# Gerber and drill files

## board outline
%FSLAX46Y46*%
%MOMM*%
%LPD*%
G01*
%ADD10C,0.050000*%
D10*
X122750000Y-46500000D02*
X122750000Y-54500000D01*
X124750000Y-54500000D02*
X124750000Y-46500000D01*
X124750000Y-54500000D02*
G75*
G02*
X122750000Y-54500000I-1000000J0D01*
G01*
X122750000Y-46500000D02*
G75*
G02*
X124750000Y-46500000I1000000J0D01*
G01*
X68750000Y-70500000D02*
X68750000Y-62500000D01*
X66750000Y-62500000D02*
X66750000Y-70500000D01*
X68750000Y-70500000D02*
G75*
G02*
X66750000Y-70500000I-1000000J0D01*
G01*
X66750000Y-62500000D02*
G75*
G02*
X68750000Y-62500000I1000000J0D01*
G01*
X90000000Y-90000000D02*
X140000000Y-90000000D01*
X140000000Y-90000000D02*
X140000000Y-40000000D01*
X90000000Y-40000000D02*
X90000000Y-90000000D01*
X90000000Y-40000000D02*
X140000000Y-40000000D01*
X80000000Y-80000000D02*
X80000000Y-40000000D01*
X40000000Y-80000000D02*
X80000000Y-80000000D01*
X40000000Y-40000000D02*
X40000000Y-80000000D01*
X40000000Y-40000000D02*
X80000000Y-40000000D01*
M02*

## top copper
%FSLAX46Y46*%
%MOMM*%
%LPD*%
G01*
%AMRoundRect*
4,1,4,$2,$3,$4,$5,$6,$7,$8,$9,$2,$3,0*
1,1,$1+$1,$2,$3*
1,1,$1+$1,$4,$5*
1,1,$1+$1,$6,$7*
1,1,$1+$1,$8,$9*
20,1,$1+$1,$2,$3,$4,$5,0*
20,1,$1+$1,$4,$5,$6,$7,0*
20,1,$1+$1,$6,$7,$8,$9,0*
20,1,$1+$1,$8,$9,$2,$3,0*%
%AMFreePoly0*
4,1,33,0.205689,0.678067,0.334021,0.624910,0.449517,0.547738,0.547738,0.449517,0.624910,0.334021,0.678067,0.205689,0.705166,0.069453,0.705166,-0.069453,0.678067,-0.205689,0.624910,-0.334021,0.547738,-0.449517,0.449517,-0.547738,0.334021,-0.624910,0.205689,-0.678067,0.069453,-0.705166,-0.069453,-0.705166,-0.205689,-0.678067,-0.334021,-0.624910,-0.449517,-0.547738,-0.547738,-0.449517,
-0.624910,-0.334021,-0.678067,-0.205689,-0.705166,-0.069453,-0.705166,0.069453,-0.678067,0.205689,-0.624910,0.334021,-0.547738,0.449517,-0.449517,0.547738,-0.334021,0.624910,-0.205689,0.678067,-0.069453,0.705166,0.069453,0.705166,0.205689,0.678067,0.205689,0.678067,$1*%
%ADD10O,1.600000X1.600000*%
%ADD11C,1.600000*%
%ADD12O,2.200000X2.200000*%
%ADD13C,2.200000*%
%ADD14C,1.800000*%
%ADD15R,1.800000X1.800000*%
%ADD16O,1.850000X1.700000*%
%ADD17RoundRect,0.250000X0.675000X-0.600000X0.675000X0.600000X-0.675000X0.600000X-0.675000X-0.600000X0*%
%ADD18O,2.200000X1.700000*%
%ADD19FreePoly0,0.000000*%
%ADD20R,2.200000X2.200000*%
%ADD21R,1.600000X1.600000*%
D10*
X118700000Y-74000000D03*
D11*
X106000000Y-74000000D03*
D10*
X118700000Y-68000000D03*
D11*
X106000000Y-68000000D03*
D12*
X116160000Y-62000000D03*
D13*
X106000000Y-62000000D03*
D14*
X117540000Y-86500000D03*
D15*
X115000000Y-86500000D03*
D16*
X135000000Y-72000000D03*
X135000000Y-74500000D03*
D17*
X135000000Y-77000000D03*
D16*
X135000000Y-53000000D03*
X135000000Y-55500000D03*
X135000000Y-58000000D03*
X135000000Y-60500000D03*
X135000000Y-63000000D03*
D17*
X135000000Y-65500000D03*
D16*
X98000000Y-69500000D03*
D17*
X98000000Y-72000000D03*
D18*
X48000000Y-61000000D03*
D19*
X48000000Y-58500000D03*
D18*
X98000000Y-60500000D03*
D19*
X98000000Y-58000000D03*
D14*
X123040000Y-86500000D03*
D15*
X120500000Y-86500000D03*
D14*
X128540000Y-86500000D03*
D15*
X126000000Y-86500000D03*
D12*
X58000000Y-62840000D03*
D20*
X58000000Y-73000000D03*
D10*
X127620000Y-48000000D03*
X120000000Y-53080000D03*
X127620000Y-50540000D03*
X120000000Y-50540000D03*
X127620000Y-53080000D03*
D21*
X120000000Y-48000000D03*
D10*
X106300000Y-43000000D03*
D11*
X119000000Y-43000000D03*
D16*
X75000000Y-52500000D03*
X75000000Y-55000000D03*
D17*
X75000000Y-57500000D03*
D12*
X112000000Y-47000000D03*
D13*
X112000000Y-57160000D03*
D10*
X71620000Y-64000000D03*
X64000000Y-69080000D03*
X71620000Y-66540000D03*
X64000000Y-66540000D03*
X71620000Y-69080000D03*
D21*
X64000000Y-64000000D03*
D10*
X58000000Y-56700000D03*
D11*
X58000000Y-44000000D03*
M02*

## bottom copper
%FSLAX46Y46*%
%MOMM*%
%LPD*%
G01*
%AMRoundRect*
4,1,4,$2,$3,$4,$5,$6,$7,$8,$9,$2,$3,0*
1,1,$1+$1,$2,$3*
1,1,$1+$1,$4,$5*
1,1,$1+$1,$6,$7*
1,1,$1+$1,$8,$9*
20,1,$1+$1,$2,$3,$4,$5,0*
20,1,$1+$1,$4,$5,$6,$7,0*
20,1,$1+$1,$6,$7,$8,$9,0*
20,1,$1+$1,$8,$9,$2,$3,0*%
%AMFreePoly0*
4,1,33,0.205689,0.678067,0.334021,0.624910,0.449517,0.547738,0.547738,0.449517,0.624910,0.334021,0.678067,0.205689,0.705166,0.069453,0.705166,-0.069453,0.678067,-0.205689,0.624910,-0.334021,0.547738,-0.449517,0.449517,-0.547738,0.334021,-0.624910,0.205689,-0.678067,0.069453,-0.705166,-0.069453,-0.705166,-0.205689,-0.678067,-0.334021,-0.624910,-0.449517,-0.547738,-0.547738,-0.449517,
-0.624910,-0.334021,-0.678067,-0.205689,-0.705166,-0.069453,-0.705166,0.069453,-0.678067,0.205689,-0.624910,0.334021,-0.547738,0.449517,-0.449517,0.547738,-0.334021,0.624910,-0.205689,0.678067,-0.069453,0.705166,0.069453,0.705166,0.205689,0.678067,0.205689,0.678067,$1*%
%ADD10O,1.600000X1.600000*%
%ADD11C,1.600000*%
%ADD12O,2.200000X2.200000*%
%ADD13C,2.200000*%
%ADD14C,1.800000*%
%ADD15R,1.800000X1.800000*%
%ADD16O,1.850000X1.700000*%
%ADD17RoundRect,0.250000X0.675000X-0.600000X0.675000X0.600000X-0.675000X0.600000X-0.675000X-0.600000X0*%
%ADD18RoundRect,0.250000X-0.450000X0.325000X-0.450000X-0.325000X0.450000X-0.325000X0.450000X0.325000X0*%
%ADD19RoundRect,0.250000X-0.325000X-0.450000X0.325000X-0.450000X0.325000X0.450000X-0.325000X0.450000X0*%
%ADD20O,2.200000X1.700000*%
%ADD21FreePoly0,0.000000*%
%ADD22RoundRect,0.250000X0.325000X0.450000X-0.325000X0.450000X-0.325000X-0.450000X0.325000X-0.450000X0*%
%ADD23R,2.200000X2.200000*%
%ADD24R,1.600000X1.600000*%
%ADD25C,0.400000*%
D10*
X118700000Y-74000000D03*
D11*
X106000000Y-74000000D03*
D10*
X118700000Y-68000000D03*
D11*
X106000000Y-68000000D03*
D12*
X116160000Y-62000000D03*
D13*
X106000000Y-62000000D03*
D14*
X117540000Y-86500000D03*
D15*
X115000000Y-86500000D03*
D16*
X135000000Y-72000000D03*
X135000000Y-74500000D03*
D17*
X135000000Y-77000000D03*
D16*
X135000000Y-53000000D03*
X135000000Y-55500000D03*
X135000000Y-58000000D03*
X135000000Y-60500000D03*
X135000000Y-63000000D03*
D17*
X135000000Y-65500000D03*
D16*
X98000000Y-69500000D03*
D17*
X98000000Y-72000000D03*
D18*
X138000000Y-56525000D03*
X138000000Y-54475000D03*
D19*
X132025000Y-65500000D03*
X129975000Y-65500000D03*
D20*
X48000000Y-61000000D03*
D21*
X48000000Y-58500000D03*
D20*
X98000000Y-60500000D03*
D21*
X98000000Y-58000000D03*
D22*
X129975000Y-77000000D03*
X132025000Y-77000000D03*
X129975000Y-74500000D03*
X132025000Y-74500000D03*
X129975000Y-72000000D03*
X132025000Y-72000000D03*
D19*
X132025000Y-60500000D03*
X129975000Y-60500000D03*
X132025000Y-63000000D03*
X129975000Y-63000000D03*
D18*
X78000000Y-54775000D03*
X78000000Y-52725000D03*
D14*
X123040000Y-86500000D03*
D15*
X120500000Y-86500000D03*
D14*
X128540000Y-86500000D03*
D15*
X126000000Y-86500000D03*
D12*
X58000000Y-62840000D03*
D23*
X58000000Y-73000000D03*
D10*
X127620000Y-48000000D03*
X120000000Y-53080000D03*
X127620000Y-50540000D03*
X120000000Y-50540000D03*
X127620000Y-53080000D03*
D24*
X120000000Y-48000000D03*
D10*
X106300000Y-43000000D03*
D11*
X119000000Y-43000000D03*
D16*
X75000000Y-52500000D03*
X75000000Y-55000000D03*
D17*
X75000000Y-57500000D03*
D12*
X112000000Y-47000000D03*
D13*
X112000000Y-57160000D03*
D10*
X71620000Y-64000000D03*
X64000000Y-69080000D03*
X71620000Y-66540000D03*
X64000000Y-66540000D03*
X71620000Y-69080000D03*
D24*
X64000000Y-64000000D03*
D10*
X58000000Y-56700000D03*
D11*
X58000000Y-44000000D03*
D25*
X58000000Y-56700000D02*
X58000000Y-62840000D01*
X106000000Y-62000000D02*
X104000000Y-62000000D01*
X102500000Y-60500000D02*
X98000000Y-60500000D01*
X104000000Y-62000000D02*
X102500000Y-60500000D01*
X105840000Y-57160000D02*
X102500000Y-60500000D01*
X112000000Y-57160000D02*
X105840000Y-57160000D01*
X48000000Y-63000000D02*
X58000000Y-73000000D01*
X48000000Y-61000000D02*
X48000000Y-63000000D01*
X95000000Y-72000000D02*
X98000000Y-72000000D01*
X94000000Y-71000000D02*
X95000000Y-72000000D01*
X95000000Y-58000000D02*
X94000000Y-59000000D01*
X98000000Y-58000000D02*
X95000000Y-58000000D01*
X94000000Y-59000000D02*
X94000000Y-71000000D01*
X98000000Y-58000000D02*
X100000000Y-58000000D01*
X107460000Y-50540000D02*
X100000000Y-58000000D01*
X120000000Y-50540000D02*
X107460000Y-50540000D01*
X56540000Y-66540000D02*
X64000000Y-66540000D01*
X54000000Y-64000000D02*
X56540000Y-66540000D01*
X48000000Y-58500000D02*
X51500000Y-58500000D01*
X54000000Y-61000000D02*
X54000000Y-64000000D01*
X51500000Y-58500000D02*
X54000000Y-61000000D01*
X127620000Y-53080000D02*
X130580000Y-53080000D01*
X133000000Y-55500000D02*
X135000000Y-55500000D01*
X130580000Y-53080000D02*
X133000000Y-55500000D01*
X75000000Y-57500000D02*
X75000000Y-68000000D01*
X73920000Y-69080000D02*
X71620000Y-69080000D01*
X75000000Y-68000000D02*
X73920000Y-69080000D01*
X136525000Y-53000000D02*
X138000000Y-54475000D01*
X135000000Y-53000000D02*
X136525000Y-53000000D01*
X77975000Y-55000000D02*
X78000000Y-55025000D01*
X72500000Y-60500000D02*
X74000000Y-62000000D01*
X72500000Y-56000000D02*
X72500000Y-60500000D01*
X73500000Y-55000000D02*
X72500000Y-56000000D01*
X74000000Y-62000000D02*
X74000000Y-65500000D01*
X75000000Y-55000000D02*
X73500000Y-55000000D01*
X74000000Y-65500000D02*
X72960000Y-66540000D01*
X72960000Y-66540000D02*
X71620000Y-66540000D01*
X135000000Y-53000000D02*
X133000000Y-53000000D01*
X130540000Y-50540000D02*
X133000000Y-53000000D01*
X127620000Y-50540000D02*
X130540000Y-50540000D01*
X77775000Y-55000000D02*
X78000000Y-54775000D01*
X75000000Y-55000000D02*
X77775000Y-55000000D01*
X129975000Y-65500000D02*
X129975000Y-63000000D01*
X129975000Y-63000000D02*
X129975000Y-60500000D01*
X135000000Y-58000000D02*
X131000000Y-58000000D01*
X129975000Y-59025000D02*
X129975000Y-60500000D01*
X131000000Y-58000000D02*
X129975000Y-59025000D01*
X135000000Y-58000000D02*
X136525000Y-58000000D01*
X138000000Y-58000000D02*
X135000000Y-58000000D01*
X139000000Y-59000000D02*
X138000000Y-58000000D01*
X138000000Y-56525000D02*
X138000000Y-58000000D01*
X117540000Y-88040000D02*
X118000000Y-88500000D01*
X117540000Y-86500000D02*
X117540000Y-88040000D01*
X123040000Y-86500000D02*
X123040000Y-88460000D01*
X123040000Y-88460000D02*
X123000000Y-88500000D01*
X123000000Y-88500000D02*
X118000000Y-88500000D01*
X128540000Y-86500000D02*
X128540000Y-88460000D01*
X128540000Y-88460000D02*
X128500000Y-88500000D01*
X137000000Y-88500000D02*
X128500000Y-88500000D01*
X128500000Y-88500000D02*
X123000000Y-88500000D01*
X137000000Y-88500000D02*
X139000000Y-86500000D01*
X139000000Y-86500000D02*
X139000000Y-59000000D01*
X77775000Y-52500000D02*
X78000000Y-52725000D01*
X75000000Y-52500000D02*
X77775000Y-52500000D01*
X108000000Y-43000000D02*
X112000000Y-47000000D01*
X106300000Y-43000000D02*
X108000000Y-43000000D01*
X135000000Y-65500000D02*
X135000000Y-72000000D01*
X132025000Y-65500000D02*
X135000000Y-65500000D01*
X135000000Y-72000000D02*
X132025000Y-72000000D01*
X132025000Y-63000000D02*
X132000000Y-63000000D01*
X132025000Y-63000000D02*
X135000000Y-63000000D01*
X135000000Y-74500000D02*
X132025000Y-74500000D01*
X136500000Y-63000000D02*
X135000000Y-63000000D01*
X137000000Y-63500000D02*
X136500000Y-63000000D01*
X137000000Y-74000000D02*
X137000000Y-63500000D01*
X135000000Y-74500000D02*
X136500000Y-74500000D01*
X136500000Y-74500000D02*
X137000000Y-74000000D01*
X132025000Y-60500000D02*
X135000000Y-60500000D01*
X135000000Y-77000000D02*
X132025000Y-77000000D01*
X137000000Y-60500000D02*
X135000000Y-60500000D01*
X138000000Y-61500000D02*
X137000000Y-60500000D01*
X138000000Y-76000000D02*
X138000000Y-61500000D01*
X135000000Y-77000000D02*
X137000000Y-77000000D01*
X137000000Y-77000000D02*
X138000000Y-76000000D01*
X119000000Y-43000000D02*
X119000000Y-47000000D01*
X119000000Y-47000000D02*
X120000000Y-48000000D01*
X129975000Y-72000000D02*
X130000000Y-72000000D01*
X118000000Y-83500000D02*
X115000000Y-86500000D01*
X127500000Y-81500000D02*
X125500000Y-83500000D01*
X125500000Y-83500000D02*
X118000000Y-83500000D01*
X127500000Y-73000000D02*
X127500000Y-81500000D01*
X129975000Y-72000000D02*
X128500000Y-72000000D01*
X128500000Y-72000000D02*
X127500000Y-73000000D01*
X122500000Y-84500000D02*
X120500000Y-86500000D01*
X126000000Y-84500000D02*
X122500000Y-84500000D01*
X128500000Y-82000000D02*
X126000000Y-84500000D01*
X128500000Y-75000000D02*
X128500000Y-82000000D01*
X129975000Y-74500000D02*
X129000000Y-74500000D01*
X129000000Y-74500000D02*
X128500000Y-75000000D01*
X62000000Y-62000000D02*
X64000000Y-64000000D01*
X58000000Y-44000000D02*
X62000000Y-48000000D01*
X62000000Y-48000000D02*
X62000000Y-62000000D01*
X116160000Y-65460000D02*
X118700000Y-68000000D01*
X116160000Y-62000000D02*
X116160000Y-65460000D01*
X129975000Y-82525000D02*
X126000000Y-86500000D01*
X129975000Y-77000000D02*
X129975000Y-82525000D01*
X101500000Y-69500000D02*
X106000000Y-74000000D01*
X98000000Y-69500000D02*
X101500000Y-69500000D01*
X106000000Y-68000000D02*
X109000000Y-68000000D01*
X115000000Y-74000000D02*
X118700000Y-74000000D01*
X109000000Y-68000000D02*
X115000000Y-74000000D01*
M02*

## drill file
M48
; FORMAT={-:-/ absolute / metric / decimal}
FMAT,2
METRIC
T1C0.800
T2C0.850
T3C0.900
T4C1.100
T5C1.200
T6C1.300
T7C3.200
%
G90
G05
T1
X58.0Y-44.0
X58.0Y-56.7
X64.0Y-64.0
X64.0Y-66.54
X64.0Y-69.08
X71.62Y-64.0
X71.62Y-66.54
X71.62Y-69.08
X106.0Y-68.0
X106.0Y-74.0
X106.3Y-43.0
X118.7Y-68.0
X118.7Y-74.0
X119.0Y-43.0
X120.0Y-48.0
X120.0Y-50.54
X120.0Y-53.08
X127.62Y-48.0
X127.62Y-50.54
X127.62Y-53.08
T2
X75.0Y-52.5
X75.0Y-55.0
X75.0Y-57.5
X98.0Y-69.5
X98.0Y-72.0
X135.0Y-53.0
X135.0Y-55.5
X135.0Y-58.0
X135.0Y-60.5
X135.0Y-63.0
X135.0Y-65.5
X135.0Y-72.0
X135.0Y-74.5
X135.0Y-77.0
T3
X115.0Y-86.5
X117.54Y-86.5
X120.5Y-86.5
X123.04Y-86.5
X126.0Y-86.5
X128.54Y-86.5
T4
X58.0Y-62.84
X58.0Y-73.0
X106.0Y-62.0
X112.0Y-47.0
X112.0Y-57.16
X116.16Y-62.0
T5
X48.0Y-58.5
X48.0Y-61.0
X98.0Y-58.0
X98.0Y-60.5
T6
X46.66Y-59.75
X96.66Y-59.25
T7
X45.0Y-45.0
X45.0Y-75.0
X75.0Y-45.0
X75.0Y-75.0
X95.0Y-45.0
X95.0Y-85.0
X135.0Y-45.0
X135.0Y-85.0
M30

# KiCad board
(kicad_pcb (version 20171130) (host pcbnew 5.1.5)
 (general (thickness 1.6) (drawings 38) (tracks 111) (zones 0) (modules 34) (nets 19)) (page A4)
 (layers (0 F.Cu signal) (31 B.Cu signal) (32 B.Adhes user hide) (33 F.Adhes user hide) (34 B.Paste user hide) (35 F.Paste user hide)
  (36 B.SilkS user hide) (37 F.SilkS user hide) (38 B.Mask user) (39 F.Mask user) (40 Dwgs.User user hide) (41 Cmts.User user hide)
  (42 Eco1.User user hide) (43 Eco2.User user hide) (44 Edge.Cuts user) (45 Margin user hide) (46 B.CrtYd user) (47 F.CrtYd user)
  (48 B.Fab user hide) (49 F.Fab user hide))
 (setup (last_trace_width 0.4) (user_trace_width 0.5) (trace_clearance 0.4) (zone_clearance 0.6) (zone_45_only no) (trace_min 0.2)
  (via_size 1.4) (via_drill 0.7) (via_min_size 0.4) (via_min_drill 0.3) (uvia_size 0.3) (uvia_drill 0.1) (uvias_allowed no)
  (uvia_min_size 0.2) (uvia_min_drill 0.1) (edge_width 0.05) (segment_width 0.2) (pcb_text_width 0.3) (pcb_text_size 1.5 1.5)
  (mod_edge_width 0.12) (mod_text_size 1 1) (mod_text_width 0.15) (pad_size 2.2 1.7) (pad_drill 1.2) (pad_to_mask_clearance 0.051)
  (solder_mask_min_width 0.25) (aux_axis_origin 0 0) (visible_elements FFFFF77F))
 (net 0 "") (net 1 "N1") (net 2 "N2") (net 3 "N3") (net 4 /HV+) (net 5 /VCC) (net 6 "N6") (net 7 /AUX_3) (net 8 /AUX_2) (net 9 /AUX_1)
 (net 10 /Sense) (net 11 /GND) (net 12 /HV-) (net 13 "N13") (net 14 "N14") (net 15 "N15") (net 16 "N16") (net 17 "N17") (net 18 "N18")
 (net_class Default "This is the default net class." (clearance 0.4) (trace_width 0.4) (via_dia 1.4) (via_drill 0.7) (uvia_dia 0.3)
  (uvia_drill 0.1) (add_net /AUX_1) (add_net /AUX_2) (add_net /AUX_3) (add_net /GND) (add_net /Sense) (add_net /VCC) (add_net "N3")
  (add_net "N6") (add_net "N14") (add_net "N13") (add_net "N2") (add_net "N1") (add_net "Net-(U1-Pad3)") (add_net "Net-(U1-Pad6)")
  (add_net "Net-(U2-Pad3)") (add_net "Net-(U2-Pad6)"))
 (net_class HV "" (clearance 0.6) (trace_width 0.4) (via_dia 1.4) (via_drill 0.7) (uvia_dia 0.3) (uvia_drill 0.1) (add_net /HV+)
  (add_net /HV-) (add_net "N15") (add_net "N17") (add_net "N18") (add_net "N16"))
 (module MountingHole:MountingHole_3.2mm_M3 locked (layer F.Cu) (at 45 45) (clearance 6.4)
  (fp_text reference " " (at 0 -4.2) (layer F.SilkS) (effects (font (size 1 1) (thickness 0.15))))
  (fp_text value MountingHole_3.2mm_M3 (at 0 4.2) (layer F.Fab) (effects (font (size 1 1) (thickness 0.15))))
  (pad 1 np_thru_hole circle (at 0 0) (size 3.2 3.2) (drill 3.2) (layers *.Cu *.Mask)))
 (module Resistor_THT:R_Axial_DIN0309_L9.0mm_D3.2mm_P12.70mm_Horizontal (layer F.Cu) (at 106 74)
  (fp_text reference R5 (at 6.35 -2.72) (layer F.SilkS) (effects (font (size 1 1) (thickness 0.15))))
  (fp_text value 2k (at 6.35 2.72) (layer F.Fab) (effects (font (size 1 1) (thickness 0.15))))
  (pad 2 thru_hole oval (at 12.7 0) (size 1.6 1.6) (drill 0.8) (layers *.Cu *.Mask) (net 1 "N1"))
  (pad 1 thru_hole circle (at 0 0) (size 1.6 1.6) (drill 0.8) (layers *.Cu *.Mask) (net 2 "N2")))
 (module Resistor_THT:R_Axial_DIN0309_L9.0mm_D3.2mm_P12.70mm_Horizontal (layer F.Cu) (at 106 68)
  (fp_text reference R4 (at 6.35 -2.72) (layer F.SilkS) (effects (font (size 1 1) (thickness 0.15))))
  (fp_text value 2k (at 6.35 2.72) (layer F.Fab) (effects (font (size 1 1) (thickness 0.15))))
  (pad 2 thru_hole oval (at 12.7 0) (size 1.6 1.6) (drill 0.8) (layers *.Cu *.Mask) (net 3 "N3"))
  (pad 1 thru_hole circle (at 0 0) (size 1.6 1.6) (drill 0.8) (layers *.Cu *.Mask) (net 1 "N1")))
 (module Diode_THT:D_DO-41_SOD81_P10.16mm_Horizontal (layer F.Cu) (at 106 62)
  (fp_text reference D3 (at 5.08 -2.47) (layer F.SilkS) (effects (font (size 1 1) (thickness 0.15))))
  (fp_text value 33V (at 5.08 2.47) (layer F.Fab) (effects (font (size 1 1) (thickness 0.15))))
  (pad 2 thru_hole oval (at 10.16 0) (size 2.2 2.2) (drill 1.1) (layers *.Cu *.Mask) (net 3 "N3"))
  (pad 1 thru_hole circle (at 0 0) (size 2.2 2.2) (drill 1.1) (layers *.Cu *.Mask) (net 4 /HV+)))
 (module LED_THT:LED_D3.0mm (layer F.Cu) (at 115 86.5)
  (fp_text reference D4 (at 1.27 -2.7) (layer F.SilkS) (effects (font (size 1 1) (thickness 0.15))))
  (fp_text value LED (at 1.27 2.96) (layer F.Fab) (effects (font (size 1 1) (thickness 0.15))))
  (pad 2 thru_hole circle (at 2.54 0) (size 1.8 1.8) (drill 0.9) (layers *.Cu *.Mask) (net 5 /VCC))
  (pad 1 thru_hole rect (at 0 0) (size 1.8 1.8) (drill 0.9) (layers *.Cu *.Mask) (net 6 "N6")))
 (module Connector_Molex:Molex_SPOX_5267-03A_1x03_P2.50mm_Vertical (layer F.Cu) (at 135 77 90)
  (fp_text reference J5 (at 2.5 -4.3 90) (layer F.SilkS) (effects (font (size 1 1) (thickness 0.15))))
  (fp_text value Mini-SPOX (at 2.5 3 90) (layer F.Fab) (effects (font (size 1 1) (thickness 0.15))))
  (pad 3 thru_hole oval (at 5 0 90) (size 1.7 1.85) (drill 0.85) (layers *.Cu *.Mask) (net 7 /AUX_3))
  (pad 2 thru_hole oval (at 2.5 0 90) (size 1.7 1.85) (drill 0.85) (layers *.Cu *.Mask) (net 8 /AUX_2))
  (pad 1 thru_hole roundrect (at 0 0 90) (size 1.7 1.85) (drill 0.85) (layers *.Cu *.Mask) (roundrect_rratio 0.147059) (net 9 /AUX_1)))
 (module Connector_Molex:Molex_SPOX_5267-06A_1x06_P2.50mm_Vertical (layer F.Cu) (at 135 65.5 90)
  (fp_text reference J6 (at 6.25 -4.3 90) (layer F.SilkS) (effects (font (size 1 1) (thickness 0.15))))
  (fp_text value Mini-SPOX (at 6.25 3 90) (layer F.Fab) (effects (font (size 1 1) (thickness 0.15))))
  (pad 6 thru_hole oval (at 12.5 0 90) (size 1.7 1.85) (drill 0.85) (layers *.Cu *.Mask) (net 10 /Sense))
  (pad 5 thru_hole oval (at 10 0 90) (size 1.7 1.85) (drill 0.85) (layers *.Cu *.Mask) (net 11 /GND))
  (pad 4 thru_hole oval (at 7.5 0 90) (size 1.7 1.85) (drill 0.85) (layers *.Cu *.Mask) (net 5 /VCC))
  (pad 3 thru_hole oval (at 5 0 90) (size 1.7 1.85) (drill 0.85) (layers *.Cu *.Mask) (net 9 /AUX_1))
  (pad 2 thru_hole oval (at 2.5 0 90) (size 1.7 1.85) (drill 0.85) (layers *.Cu *.Mask) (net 8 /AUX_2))
  (pad 1 thru_hole roundrect (at 0 0 90) (size 1.7 1.85) (drill 0.85) (layers *.Cu *.Mask) (roundrect_rratio 0.147059) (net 7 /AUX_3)))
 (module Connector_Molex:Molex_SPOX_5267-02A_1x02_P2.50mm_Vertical (layer F.Cu) (at 98 72 90)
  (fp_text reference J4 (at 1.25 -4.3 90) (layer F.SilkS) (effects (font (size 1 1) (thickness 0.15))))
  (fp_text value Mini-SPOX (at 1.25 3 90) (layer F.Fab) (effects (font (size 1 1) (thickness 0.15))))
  (pad 2 thru_hole oval (at 2.5 0 90) (size 1.7 1.85) (drill 0.85) (layers *.Cu *.Mask) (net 2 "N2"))
  (pad 1 thru_hole roundrect (at 0 0 90) (size 1.7 1.85) (drill 0.85) (layers *.Cu *.Mask) (roundrect_rratio 0.147059) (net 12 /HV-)))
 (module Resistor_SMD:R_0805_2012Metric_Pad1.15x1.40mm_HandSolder (layer B.Cu) (at 138 55.5 270)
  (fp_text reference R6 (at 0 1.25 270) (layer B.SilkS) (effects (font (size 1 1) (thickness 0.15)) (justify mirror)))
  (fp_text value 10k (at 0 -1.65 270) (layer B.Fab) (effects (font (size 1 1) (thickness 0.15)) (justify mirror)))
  (pad 2 smd roundrect (at 1.025 0 270) (size 1.15 1.4) (layers B.Cu B.Paste B.Mask) (roundrect_rratio 0.217391) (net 5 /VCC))
  (pad 1 smd roundrect (at -1.025 0 270) (size 1.15 1.4) (layers B.Cu B.Paste B.Mask) (roundrect_rratio 0.217391) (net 10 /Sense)))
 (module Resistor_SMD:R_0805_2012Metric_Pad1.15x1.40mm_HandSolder (layer B.Cu) (at 131 65.5)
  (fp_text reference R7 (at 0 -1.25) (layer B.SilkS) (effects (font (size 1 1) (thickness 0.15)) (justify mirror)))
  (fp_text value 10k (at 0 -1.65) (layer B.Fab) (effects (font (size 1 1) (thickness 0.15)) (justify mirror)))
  (pad 2 smd roundrect (at 1.025 0) (size 1.15 1.4) (layers B.Cu B.Paste B.Mask) (roundrect_rratio 0.217391) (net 7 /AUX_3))
  (pad 1 smd roundrect (at -1.025 0) (size 1.15 1.4) (layers B.Cu B.Paste B.Mask) (roundrect_rratio 0.217391) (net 5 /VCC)))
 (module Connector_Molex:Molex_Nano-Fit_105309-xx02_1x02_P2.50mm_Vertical (layer F.Cu) (at 48 58.5)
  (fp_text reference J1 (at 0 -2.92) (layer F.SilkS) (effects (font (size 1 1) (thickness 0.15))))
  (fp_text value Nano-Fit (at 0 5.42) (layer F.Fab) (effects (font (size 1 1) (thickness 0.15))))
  (pad "" np_thru_hole circle (at -1.34 1.25) (size 1.3 1.3) (drill 1.3) (layers *.Cu *.Mask))
  (pad 2 thru_hole oval (at 0 2.5) (size 2.2 1.7) (drill 1.2) (layers *.Cu *.Mask) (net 4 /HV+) (zone_connect 2))
  (pad 1 thru_hole custom (at 0 0) (size 1.417157 1.417157) (drill 1.2) (layers *.Cu *.Mask) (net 12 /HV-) (zone_connect 2)
   (options (clearance outline) (anchor circle)) (primitives)))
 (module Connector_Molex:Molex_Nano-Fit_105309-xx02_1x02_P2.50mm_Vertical (layer F.Cu) (at 98 58)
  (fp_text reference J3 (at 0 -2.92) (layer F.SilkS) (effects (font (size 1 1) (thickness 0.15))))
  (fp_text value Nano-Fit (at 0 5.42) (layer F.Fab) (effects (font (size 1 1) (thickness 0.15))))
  (pad "" np_thru_hole circle (at -1.34 1.25) (size 1.3 1.3) (drill 1.3) (layers *.Cu *.Mask))
  (pad 2 thru_hole oval (at 0 2.5) (size 2.2 1.7) (drill 1.2) (layers *.Cu *.Mask) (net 4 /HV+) (zone_connect 2))
  (pad 1 thru_hole custom (at 0 0) (size 1.417157 1.417157) (drill 1.2) (layers *.Cu *.Mask) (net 12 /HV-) (zone_connect 2)
   (options (clearance outline) (anchor circle)) (primitives)))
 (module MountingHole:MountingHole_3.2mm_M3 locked (layer F.Cu) (at 95 45) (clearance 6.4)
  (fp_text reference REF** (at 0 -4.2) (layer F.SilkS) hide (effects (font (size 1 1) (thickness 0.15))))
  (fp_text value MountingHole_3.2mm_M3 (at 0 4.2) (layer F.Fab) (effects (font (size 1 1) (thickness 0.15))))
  (pad 1 np_thru_hole circle (at 0 0) (size 3.2 3.2) (drill 3.2) (layers *.Cu *.Mask)))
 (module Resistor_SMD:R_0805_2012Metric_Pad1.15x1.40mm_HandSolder (layer B.Cu) (at 131 77 180)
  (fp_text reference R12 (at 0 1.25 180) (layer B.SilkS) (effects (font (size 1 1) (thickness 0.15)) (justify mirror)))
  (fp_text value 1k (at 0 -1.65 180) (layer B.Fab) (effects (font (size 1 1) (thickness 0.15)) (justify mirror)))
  (pad 2 smd roundrect (at 1.025 0 180) (size 1.15 1.4) (layers B.Cu B.Paste B.Mask) (roundrect_rratio 0.217391) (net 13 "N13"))
  (pad 1 smd roundrect (at -1.025 0 180) (size 1.15 1.4) (layers B.Cu B.Paste B.Mask) (roundrect_rratio 0.217391) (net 9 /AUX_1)))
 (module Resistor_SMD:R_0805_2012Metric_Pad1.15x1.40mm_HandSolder (layer B.Cu) (at 131 74.5 180)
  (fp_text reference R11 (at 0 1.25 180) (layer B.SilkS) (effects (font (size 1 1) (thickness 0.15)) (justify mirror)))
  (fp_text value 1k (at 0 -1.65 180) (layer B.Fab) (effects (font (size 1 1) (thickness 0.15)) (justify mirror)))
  (pad 2 smd roundrect (at 1.025 0 180) (size 1.15 1.4) (layers B.Cu B.Paste B.Mask) (roundrect_rratio 0.217391) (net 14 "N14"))
  (pad 1 smd roundrect (at -1.025 0 180) (size 1.15 1.4) (layers B.Cu B.Paste B.Mask) (roundrect_rratio 0.217391) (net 8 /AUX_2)))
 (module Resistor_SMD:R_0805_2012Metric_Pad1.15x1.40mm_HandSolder (layer B.Cu) (at 131 72 180)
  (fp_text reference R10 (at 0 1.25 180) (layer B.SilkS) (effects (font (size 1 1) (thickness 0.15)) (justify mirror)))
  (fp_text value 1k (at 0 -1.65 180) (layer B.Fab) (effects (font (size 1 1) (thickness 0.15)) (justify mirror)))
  (pad 2 smd roundrect (at 1.025 0 180) (size 1.15 1.4) (layers B.Cu B.Paste B.Mask) (roundrect_rratio 0.217391) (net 6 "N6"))
  (pad 1 smd roundrect (at -1.025 0 180) (size 1.15 1.4) (layers B.Cu B.Paste B.Mask) (roundrect_rratio 0.217391) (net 7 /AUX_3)))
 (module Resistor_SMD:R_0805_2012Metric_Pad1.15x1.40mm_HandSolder (layer B.Cu) (at 131 60.5)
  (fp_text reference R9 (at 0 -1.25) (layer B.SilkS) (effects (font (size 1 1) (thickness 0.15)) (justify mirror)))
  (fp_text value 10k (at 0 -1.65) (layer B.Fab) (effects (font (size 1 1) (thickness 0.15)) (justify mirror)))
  (pad 2 smd roundrect (at 1.025 0) (size 1.15 1.4) (layers B.Cu B.Paste B.Mask) (roundrect_rratio 0.217391) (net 9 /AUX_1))
  (pad 1 smd roundrect (at -1.025 0) (size 1.15 1.4) (layers B.Cu B.Paste B.Mask) (roundrect_rratio 0.217391) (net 5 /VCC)))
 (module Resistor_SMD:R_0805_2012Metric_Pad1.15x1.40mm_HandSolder (layer B.Cu) (at 131 63)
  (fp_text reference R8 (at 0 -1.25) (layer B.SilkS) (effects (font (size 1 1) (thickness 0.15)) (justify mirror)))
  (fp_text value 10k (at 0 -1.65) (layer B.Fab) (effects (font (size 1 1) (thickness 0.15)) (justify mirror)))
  (pad 2 smd roundrect (at 1.025 0) (size 1.15 1.4) (layers B.Cu B.Paste B.Mask) (roundrect_rratio 0.217391) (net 8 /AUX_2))
  (pad 1 smd roundrect (at -1.025 0) (size 1.15 1.4) (layers B.Cu B.Paste B.Mask) (roundrect_rratio 0.217391) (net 5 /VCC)))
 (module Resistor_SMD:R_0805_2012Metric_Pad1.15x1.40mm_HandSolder (layer B.Cu) (at 78 53.75 270)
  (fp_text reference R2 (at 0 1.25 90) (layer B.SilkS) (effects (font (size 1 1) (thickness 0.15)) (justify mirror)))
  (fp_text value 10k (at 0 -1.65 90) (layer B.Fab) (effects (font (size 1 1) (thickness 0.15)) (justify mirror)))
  (pad 2 smd roundrect (at 1.025 0 270) (size 1.15 1.4) (layers B.Cu B.Paste B.Mask) (roundrect_rratio 0.217391) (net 10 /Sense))
  (pad 1 smd roundrect (at -1.025 0 270) (size 1.15 1.4) (layers B.Cu B.Paste B.Mask) (roundrect_rratio 0.217391) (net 5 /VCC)))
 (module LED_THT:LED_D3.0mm (layer F.Cu) (at 120.5 86.5)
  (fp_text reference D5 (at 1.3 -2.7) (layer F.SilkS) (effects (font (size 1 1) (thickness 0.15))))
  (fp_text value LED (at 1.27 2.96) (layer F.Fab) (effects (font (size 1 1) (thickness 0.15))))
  (pad 2 thru_hole circle (at 2.54 0) (size 1.8 1.8) (drill 0.9) (layers *.Cu *.Mask) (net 5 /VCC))
  (pad 1 thru_hole rect (at 0 0) (size 1.8 1.8) (drill 0.9) (layers *.Cu *.Mask) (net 14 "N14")))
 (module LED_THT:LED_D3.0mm (layer F.Cu) (at 126 86.5)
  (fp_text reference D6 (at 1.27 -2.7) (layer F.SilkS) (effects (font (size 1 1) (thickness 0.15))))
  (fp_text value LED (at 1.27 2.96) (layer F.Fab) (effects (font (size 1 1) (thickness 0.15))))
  (pad 2 thru_hole circle (at 2.54 0) (size 1.8 1.8) (drill 0.9) (layers *.Cu *.Mask) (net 5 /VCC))
  (pad 1 thru_hole rect (at 0 0) (size 1.8 1.8) (drill 0.9) (layers *.Cu *.Mask) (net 13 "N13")))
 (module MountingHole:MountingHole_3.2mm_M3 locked (layer F.Cu) (at 135 85)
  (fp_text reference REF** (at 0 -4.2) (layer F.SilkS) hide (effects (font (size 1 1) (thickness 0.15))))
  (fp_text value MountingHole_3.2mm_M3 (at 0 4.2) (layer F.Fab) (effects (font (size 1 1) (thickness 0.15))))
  (pad 1 np_thru_hole circle (at 0 0) (size 3.2 3.2) (drill 3.2) (layers *.Cu *.Mask)))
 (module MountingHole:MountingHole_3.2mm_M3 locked (layer F.Cu) (at 75 75)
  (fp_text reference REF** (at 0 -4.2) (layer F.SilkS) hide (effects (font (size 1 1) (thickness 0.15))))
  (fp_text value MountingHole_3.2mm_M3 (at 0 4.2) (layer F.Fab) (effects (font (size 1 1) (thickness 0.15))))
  (pad 1 np_thru_hole circle (at 0 0) (size 3.2 3.2) (drill 3.2) (layers *.Cu *.Mask)))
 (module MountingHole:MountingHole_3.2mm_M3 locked (layer F.Cu) (at 95 85) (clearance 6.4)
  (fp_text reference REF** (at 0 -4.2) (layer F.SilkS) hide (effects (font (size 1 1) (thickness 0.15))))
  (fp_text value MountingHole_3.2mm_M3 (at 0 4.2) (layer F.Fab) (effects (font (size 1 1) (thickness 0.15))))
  (pad 1 np_thru_hole circle (at 0 0) (size 3.2 3.2) (drill 3.2) (layers *.Cu *.Mask)))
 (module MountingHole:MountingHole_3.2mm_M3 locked (layer F.Cu) (at 135 45)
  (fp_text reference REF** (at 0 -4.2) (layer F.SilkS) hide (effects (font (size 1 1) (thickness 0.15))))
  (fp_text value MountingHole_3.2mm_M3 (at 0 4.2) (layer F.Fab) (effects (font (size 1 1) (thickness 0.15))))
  (pad 1 np_thru_hole circle (at 0 0) (size 3.2 3.2) (drill 3.2) (layers *.Cu *.Mask)))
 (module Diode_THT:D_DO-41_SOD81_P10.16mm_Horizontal (layer F.Cu) (at 58 73 90)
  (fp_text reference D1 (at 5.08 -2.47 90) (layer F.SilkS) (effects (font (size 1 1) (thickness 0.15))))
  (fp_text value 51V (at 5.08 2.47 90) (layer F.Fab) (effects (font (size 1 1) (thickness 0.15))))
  (pad 2 thru_hole oval (at 10.16 0 90) (size 2.2 2.2) (drill 1.1) (layers *.Cu *.Mask) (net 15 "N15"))
  (pad 1 thru_hole rect (at 0 0 90) (size 2.2 2.2) (drill 1.1) (layers *.Cu *.Mask) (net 4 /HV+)))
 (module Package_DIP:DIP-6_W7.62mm (layer F.Cu) (at 120 48)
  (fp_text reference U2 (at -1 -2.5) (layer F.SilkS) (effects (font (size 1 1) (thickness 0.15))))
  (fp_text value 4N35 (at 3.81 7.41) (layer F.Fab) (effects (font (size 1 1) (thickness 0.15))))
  (pad 6 thru_hole oval (at 7.62 0) (size 1.6 1.6) (drill 0.8) (layers *.Cu *.Mask))
  (pad 3 thru_hole oval (at 0 5.08) (size 1.6 1.6) (drill 0.8) (layers *.Cu *.Mask))
  (pad 5 thru_hole oval (at 7.62 2.54) (size 1.6 1.6) (drill 0.8) (layers *.Cu *.Mask) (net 10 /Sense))
  (pad 2 thru_hole oval (at 0 2.54) (size 1.6 1.6) (drill 0.8) (layers *.Cu *.Mask) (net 12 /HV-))
  (pad 4 thru_hole oval (at 7.62 5.08) (size 1.6 1.6) (drill 0.8) (layers *.Cu *.Mask) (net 11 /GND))
  (pad 1 thru_hole rect (at 0 0) (size 1.6 1.6) (drill 0.8) (layers *.Cu *.Mask) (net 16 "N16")))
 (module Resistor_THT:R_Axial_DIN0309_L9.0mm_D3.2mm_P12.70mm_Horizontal (layer F.Cu) (at 119 43 180)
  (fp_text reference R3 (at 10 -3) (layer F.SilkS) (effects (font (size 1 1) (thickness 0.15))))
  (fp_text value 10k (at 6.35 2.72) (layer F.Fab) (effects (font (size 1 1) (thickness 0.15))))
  (pad 2 thru_hole oval (at 12.7 0 180) (size 1.6 1.6) (drill 0.8) (layers *.Cu *.Mask) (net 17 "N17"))
  (pad 1 thru_hole circle (at 0 0 180) (size 1.6 1.6) (drill 0.8) (layers *.Cu *.Mask) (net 16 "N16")))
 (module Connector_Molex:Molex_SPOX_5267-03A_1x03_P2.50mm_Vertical (layer F.Cu) (at 75 57.5 90)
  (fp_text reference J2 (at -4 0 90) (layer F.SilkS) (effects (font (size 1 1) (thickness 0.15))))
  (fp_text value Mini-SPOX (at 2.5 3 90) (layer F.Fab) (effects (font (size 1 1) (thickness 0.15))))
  (pad 3 thru_hole oval (at 5 0 90) (size 1.7 1.85) (drill 0.85) (layers *.Cu *.Mask) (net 5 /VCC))
  (pad 2 thru_hole oval (at 2.5 0 90) (size 1.7 1.85) (drill 0.85) (layers *.Cu *.Mask) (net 10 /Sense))
  (pad 1 thru_hole roundrect (at 0 0 90) (size 1.7 1.85) (drill 0.85) (layers *.Cu *.Mask) (roundrect_rratio 0.147059) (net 11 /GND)))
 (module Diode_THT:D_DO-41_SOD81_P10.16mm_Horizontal (layer F.Cu) (at 112 57.16 90)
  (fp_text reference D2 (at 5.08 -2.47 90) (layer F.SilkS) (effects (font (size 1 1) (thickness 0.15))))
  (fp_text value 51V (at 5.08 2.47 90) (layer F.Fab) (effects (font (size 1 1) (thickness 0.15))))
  (pad 2 thru_hole oval (at 10.16 0 90) (size 2.2 2.2) (drill 1.1) (layers *.Cu *.Mask) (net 17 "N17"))
  (pad 1 thru_hole circle (at 0 0 90) (size 2.2 2.2) (drill 1.1) (layers *.Cu *.Mask) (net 4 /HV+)))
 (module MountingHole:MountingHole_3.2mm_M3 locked (layer F.Cu) (at 75 45)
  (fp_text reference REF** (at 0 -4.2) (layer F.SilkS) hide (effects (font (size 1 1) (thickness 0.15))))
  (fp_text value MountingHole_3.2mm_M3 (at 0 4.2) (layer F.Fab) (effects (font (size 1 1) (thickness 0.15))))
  (pad 1 np_thru_hole circle (at 0 0) (size 3.2 3.2) (drill 3.2) (layers *.Cu *.Mask)))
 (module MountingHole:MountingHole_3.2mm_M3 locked (layer F.Cu) (at 45 75) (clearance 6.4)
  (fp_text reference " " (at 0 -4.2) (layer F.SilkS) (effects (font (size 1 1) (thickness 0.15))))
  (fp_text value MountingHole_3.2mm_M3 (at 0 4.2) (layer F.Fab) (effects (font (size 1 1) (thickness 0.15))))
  (pad 1 np_thru_hole circle (at 0 0) (size 3.2 3.2) (drill 3.2) (layers *.Cu *.Mask)))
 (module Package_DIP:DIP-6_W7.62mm (layer F.Cu) (at 64 64)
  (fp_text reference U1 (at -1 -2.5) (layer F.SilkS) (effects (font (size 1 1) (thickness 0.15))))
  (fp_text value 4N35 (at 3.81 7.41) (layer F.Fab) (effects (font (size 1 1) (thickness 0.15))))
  (pad 6 thru_hole oval (at 7.62 0) (size 1.6 1.6) (drill 0.8) (layers *.Cu *.Mask))
  (pad 3 thru_hole oval (at 0 5.08) (size 1.6 1.6) (drill 0.8) (layers *.Cu *.Mask))
  (pad 5 thru_hole oval (at 7.62 2.54) (size 1.6 1.6) (drill 0.8) (layers *.Cu *.Mask) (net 10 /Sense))
  (pad 2 thru_hole oval (at 0 2.54) (size 1.6 1.6) (drill 0.8) (layers *.Cu *.Mask) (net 12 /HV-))
  (pad 4 thru_hole oval (at 7.62 5.08) (size 1.6 1.6) (drill 0.8) (layers *.Cu *.Mask) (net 11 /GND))
  (pad 1 thru_hole rect (at 0 0) (size 1.6 1.6) (drill 0.8) (layers *.Cu *.Mask) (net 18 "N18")))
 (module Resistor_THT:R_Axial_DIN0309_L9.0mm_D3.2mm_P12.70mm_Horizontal (layer F.Cu) (at 58 44 270)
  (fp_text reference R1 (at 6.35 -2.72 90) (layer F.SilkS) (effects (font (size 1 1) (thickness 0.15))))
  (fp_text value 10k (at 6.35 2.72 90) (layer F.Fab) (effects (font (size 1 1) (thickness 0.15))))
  (pad 2 thru_hole oval (at 12.7 0 270) (size 1.6 1.6) (drill 0.8) (layers *.Cu *.Mask) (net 15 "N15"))
  (pad 1 thru_hole circle (at 0 0 270) (size 1.6 1.6) (drill 0.8) (layers *.Cu *.Mask) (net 18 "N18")))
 (gr_line (start 122.75 46.5) (end 122.75 54.5) (layer Edge.Cuts) (width 0.05))
 (gr_line (start 124.75 54.5) (end 124.75 46.5) (layer Edge.Cuts) (width 0.05))
 (gr_arc (start 123.75 54.5) (end 122.75 54.5) (angle -180) (layer Edge.Cuts) (width 0.05))
 (gr_arc (start 123.75 46.5) (end 124.75 46.5) (angle -180) (layer Edge.Cuts) (width 0.05))
 (gr_line (start 68.75 70.5) (end 68.75 62.5) (layer Edge.Cuts) (width 0.05))
 (gr_line (start 66.75 62.5) (end 66.75 70.5) (layer Edge.Cuts) (width 0.05))
 (gr_arc (start 67.75 70.5) (end 66.75 70.5) (angle -180) (layer Edge.Cuts) (width 0.05))
 (gr_arc (start 67.75 62.5) (end 68.75 62.5) (angle -180) (layer Edge.Cuts) (width 0.05))
 (gr_line (start 90 90) (end 140 90) (layer Edge.Cuts) (width 0.05))
 (gr_line (start 140 90) (end 140 40) (layer Edge.Cuts) (width 0.05))
 (gr_line (start 90 40) (end 90 90) (layer Edge.Cuts) (width 0.05))
 (gr_line (start 90 40) (end 140 40) (layer Edge.Cuts) (width 0.05))
 (gr_line (start 80 80) (end 80 40) (layer Edge.Cuts) (width 0.05))
 (gr_line (start 40 80) (end 80 80) (layer Edge.Cuts) (width 0.05))
 (gr_line (start 40 40) (end 40 80) (layer Edge.Cuts) (width 0.05))
 (gr_line (start 40 40) (end 80 40) (layer Edge.Cuts) (width 0.05))
 (segment (start 58 56.7) (end 58 62.84) (width 0.4) (layer B.Cu) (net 15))
 (segment (start 106 62) (end 104 62) (width 0.4) (layer B.Cu) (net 4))
 (segment (start 102.5 60.5) (end 98 60.5) (width 0.4) (layer B.Cu) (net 4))
 (segment (start 104 62) (end 102.5 60.5) (width 0.4) (layer B.Cu) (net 4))
 (segment (start 105.84 57.16) (end 102.5 60.5) (width 0.4) (layer B.Cu) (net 4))
 (segment (start 112 57.16) (end 105.84 57.16) (width 0.4) (layer B.Cu) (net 4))
 (segment (start 48 63) (end 58 73) (width 0.4) (layer B.Cu) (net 4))
 (segment (start 48 61) (end 48 63) (width 0.4) (layer B.Cu) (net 4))
 (segment (start 95 72) (end 98 72) (width 0.4) (layer B.Cu) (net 12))
 (segment (start 94 71) (end 95 72) (width 0.4) (layer B.Cu) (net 12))
 (segment (start 95 58) (end 94 59) (width 0.4) (layer B.Cu) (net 12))
 (segment (start 98 58) (end 95 58) (width 0.4) (layer B.Cu) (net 12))
 (segment (start 94 59) (end 94 71) (width 0.4) (layer B.Cu) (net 12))
 (segment (start 98 58) (end 100 58) (width 0.4) (layer B.Cu) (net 12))
 (segment (start 107.46 50.54) (end 100 58) (width 0.4) (layer B.Cu) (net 12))
 (segment (start 120 50.54) (end 107.46 50.54) (width 0.4) (layer B.Cu) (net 12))
 (segment (start 56.54 66.54) (end 64 66.54) (width 0.4) (layer B.Cu) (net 12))
 (segment (start 54 64) (end 56.54 66.54) (width 0.4) (layer B.Cu) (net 12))
 (segment (start 48 58.5) (end 51.5 58.5) (width 0.4) (layer B.Cu) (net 12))
 (segment (start 54 61) (end 54 64) (width 0.4) (layer B.Cu) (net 12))
 (segment (start 51.5 58.5) (end 54 61) (width 0.4) (layer B.Cu) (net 12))
 (segment (start 127.62 53.08) (end 130.58 53.08) (width 0.4) (layer B.Cu) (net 11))
 (segment (start 133 55.5) (end 135 55.5) (width 0.4) (layer B.Cu) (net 11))
 (segment (start 130.58 53.08) (end 133 55.5) (width 0.4) (layer B.Cu) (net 11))
 (segment (start 75 57.5) (end 75 68) (width 0.4) (layer B.Cu) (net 11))
 (segment (start 73.92 69.08) (end 71.62 69.08) (width 0.4) (layer B.Cu) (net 11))
 (segment (start 75 68) (end 73.92 69.08) (width 0.4) (layer B.Cu) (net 11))
 (segment (start 136.525 53) (end 138 54.475) (width 0.4) (layer B.Cu) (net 10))
 (segment (start 135 53) (end 136.525 53) (width 0.4) (layer B.Cu) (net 10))
 (segment (start 77.975 55) (end 78 55.025) (width 0.4) (layer B.Cu) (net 10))
 (segment (start 72.5 60.5) (end 74 62) (width 0.4) (layer B.Cu) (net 10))
 (segment (start 72.5 56) (end 72.5 60.5) (width 0.4) (layer B.Cu) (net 10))
 (segment (start 73.5 55) (end 72.5 56) (width 0.4) (layer B.Cu) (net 10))
 (segment (start 74 62) (end 74 65.5) (width 0.4) (layer B.Cu) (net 10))
 (segment (start 75 55) (end 73.5 55) (width 0.4) (layer B.Cu) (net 10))
 (segment (start 74 65.5) (end 72.96 66.54) (width 0.4) (layer B.Cu) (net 10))
 (segment (start 72.96 66.54) (end 71.62 66.54) (width 0.4) (layer B.Cu) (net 10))
 (segment (start 135 53) (end 133 53) (width 0.4) (layer B.Cu) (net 10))
 (segment (start 130.54 50.54) (end 133 53) (width 0.4) (layer B.Cu) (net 10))
 (segment (start 127.62 50.54) (end 130.54 50.54) (width 0.4) (layer B.Cu) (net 10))
 (segment (start 77.775 55) (end 78 54.775) (width 0.4) (layer B.Cu) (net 10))
 (segment (start 75 55) (end 77.775 55) (width 0.4) (layer B.Cu) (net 10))
 (segment (start 129.975 65.5) (end 129.975 63) (width 0.4) (layer B.Cu) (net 5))
 (segment (start 129.975 63) (end 129.975 60.5) (width 0.4) (layer B.Cu) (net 5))
 (segment (start 135 58) (end 131 58) (width 0.4) (layer B.Cu) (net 5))
 (segment (start 129.975 59.025) (end 129.975 60.5) (width 0.4) (layer B.Cu) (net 5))
 (segment (start 131 58) (end 129.975 59.025) (width 0.4) (layer B.Cu) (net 5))
 (segment (start 135 58) (end 136.525 58) (width 0.4) (layer B.Cu) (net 5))
 (segment (start 138 58) (end 135 58) (width 0.4) (layer B.Cu) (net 5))
 (segment (start 139 59) (end 138 58) (width 0.4) (layer B.Cu) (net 5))
 (segment (start 138 56.525) (end 138 58) (width 0.4) (layer B.Cu) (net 5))
 (segment (start 117.54 88.04) (end 118 88.5) (width 0.4) (layer B.Cu) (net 5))
 (segment (start 117.54 86.5) (end 117.54 88.04) (width 0.4) (layer B.Cu) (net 5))
 (segment (start 123.04 86.5) (end 123.04 88.46) (width 0.4) (layer B.Cu) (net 5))
 (segment (start 123.04 88.46) (end 123 88.5) (width 0.4) (layer B.Cu) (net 5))
 (segment (start 123 88.5) (end 118 88.5) (width 0.4) (layer B.Cu) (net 5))
 (segment (start 128.54 86.5) (end 128.54 88.46) (width 0.4) (layer B.Cu) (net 5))
 (segment (start 128.54 88.46) (end 128.5 88.5) (width 0.4) (layer B.Cu) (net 5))
 (segment (start 137 88.5) (end 128.5 88.5) (width 0.4) (layer B.Cu) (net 5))
 (segment (start 128.5 88.5) (end 123 88.5) (width 0.4) (layer B.Cu) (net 5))
 (segment (start 137 88.5) (end 139 86.5) (width 0.4) (layer B.Cu) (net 5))
 (segment (start 139 86.5) (end 139 59) (width 0.4) (layer B.Cu) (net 5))
 (segment (start 77.775 52.5) (end 78 52.725) (width 0.4) (layer B.Cu) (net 5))
 (segment (start 75 52.5) (end 77.775 52.5) (width 0.4) (layer B.Cu) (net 5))
 (segment (start 108 43) (end 112 47) (width 0.4) (layer B.Cu) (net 17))
 (segment (start 106.3 43) (end 108 43) (width 0.4) (layer B.Cu) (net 17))
 (segment (start 135 65.5) (end 135 72) (width 0.4) (layer B.Cu) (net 7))
 (segment (start 132.025 65.5) (end 135 65.5) (width 0.4) (layer B.Cu) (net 7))
 (segment (start 135 72) (end 132.025 72) (width 0.4) (layer B.Cu) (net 7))
 (segment (start 132.025 63) (end 132 63) (width 0.4) (layer B.Cu) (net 8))
 (segment (start 132.025 63) (end 135 63) (width 0.4) (layer B.Cu) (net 8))
 (segment (start 135 74.5) (end 132.025 74.5) (width 0.4) (layer B.Cu) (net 8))
 (segment (start 136.5 63) (end 135 63) (width 0.4) (layer B.Cu) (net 8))
 (segment (start 137 63.5) (end 136.5 63) (width 0.4) (layer B.Cu) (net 8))
 (segment (start 137 74) (end 137 63.5) (width 0.4) (layer B.Cu) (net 8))
 (segment (start 135 74.5) (end 136.5 74.5) (width 0.4) (layer B.Cu) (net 8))
 (segment (start 136.5 74.5) (end 137 74) (width 0.4) (layer B.Cu) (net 8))
 (segment (start 132.025 60.5) (end 135 60.5) (width 0.4) (layer B.Cu) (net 9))
 (segment (start 135 77) (end 132.025 77) (width 0.4) (layer B.Cu) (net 9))
 (segment (start 137 60.5) (end 135 60.5) (width 0.4) (layer B.Cu) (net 9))
 (segment (start 138 61.5) (end 137 60.5) (width 0.4) (layer B.Cu) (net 9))
 (segment (start 138 76) (end 138 61.5) (width 0.4) (layer B.Cu) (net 9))
 (segment (start 135 77) (end 137 77) (width 0.4) (layer B.Cu) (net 9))
 (segment (start 137 77) (end 138 76) (width 0.4) (layer B.Cu) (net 9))
 (segment (start 119 43) (end 119 47) (width 0.4) (layer B.Cu) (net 16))
 (segment (start 119 47) (end 120 48) (width 0.4) (layer B.Cu) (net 16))
 (segment (start 129.975 72) (end 130 72) (width 0.4) (layer B.Cu) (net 6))
 (segment (start 118 83.5) (end 115 86.5) (width 0.4) (layer B.Cu) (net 6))
 (segment (start 127.5 81.5) (end 125.5 83.5) (width 0.4) (layer B.Cu) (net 6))
 (segment (start 125.5 83.5) (end 118 83.5) (width 0.4) (layer B.Cu) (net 6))
 (segment (start 127.5 73) (end 127.5 81.5) (width 0.4) (layer B.Cu) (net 6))
 (segment (start 129.975 72) (end 128.5 72) (width 0.4) (layer B.Cu) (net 6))
 (segment (start 128.5 72) (end 127.5 73) (width 0.4) (layer B.Cu) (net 6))
 (segment (start 122.5 84.5) (end 120.5 86.5) (width 0.4) (layer B.Cu) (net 14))
 (segment (start 126 84.5) (end 122.5 84.5) (width 0.4) (layer B.Cu) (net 14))
 (segment (start 128.5 82) (end 126 84.5) (width 0.4) (layer B.Cu) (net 14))
 (segment (start 128.5 75) (end 128.5 82) (width 0.4) (layer B.Cu) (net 14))
 (segment (start 129.975 74.5) (end 129 74.5) (width 0.4) (layer B.Cu) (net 14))
 (segment (start 129 74.5) (end 128.5 75) (width 0.4) (layer B.Cu) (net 14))
 (segment (start 62 62) (end 64 64) (width 0.4) (layer B.Cu) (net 18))
 (segment (start 58 44) (end 62 48) (width 0.4) (layer B.Cu) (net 18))
 (segment (start 62 48) (end 62 62) (width 0.4) (layer B.Cu) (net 18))
 (segment (start 116.16 65.46) (end 118.7 68) (width 0.4) (layer B.Cu) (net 3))
 (segment (start 116.16 62) (end 116.16 65.46) (width 0.4) (layer B.Cu) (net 3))
 (segment (start 129.975 82.525) (end 126 86.5) (width 0.4) (layer B.Cu) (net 13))
 (segment (start 129.975 77) (end 129.975 82.525) (width 0.4) (layer B.Cu) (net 13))
 (segment (start 101.5 69.5) (end 106 74) (width 0.4) (layer B.Cu) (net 2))
 (segment (start 98 69.5) (end 101.5 69.5) (width 0.4) (layer B.Cu) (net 2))
 (segment (start 106 68) (end 109 68) (width 0.4) (layer B.Cu) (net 1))
 (segment (start 115 74) (end 118.7 74) (width 0.4) (layer B.Cu) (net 1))
 (segment (start 109 68) (end 115 74) (width 0.4) (layer B.Cu) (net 1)))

